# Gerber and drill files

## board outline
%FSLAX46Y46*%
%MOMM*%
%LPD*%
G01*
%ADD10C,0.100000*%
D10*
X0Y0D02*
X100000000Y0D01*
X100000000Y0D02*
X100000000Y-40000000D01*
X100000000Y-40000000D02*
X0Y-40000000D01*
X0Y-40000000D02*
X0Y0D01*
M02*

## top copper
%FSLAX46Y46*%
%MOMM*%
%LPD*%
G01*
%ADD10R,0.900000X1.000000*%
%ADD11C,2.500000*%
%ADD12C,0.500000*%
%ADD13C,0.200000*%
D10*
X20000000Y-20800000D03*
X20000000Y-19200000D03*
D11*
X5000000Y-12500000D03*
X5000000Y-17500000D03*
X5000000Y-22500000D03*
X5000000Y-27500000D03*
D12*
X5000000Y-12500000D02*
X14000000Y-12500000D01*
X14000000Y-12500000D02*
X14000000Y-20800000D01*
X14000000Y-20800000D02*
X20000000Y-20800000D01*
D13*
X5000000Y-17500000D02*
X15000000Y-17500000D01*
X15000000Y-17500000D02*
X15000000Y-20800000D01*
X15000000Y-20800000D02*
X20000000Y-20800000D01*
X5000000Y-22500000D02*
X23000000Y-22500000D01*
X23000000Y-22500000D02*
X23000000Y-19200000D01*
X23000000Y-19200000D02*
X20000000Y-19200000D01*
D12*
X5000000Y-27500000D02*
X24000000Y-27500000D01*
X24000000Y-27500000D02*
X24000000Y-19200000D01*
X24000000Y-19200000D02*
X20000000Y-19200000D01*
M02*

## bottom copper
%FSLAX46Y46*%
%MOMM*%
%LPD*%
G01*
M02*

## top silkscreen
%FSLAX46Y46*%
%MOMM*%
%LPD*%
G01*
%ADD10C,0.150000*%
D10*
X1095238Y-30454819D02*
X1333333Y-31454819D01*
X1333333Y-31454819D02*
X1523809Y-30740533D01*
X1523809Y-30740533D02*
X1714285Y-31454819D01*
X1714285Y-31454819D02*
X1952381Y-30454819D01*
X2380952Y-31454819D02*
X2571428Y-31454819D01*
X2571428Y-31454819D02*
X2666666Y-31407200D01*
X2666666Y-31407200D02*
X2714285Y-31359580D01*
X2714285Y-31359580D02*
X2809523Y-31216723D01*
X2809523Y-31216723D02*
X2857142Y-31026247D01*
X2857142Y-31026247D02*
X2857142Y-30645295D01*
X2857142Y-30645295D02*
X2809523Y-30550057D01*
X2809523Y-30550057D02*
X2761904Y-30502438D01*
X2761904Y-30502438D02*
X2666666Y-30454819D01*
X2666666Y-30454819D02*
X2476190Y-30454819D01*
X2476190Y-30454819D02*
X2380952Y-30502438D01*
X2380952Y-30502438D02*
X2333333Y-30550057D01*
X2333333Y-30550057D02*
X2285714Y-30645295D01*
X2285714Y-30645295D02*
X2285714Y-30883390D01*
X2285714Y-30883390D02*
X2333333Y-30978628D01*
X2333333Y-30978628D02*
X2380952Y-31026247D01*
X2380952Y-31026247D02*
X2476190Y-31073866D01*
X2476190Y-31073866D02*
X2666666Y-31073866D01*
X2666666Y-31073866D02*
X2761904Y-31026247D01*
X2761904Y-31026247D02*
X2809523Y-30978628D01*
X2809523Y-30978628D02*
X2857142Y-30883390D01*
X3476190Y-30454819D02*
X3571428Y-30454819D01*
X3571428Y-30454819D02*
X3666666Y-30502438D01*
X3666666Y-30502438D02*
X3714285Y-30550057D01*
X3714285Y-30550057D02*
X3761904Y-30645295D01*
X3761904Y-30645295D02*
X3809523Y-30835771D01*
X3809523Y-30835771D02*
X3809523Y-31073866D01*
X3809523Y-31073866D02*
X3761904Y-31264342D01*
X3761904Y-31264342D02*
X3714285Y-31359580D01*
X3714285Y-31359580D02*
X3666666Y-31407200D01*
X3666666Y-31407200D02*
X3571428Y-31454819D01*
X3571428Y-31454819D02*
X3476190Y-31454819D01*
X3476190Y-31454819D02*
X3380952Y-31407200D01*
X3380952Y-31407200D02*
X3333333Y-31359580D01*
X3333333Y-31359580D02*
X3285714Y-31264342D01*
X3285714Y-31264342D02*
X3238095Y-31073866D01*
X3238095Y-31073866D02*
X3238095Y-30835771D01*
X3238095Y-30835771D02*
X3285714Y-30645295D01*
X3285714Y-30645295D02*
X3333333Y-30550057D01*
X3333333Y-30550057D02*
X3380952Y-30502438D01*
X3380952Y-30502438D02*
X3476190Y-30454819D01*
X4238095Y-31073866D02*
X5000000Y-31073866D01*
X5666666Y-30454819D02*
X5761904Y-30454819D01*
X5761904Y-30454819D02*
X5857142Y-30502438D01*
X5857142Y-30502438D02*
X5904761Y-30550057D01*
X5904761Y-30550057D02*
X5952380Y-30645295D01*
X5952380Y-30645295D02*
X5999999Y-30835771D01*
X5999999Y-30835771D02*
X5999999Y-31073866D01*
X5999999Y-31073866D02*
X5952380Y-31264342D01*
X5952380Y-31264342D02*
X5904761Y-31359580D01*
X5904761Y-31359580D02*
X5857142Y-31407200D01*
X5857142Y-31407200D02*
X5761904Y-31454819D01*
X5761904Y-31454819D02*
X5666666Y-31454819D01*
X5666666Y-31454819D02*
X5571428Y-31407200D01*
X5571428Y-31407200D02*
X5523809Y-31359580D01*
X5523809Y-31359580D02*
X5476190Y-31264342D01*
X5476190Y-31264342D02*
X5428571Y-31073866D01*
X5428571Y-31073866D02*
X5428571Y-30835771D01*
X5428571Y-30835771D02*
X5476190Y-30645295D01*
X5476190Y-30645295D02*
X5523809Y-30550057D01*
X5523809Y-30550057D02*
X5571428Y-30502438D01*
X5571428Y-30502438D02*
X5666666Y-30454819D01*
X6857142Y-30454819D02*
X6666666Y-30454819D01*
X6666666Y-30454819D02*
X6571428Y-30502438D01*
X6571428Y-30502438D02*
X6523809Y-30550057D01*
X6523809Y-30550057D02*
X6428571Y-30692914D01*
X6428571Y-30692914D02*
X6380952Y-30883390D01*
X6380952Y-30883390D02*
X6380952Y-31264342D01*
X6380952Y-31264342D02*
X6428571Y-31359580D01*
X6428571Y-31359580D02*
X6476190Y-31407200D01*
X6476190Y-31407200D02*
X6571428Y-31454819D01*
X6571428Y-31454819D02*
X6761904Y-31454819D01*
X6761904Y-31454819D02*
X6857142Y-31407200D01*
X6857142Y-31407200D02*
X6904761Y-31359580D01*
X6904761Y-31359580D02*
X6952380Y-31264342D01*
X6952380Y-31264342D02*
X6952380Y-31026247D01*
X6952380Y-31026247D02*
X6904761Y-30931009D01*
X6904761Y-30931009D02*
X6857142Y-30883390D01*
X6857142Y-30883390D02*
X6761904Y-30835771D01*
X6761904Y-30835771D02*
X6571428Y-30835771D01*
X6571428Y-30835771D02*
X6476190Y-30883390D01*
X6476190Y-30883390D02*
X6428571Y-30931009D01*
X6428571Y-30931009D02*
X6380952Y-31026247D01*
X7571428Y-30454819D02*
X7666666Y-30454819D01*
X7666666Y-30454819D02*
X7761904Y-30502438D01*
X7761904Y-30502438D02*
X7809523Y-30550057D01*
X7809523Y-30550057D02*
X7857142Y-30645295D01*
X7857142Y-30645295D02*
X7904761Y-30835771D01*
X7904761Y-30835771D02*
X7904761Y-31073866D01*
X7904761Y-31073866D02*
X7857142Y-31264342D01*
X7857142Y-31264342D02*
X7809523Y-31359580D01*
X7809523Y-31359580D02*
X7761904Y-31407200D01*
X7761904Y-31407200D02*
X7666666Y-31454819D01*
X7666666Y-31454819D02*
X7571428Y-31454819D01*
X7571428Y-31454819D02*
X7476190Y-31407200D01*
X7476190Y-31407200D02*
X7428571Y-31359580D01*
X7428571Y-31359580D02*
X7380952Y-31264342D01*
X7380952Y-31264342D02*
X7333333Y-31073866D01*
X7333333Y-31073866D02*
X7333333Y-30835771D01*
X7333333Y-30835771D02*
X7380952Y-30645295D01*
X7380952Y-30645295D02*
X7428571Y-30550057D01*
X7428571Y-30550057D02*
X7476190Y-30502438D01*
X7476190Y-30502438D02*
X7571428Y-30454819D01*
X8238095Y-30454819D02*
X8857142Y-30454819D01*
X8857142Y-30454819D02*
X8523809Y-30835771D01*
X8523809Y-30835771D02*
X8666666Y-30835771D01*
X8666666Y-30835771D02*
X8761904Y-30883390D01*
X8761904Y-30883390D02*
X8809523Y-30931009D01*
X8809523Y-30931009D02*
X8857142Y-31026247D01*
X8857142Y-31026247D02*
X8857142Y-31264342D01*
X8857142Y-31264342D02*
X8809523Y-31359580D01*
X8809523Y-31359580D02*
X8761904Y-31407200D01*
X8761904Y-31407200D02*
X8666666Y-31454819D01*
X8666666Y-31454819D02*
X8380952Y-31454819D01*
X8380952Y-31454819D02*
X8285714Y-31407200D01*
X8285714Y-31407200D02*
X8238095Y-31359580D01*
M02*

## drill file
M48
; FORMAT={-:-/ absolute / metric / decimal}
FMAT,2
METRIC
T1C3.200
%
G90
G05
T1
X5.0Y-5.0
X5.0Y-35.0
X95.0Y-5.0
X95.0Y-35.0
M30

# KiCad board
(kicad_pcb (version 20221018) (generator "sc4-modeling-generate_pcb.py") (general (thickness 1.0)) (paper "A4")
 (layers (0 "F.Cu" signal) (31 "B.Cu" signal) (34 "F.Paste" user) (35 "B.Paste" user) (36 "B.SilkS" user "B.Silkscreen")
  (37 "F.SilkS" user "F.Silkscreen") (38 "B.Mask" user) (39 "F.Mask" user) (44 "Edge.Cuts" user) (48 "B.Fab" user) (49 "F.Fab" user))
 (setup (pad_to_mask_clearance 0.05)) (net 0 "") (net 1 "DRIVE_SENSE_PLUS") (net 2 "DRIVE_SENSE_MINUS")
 (gr_line (start 0.0 0.0) (end 100.0 0.0) (layer "Edge.Cuts") (width 0.1))
 (gr_line (start 100.0 0.0) (end 100.0 40.0) (layer "Edge.Cuts") (width 0.1))
 (gr_line (start 100.0 40.0) (end 0.0 40.0) (layer "Edge.Cuts") (width 0.1))
 (gr_line (start 0.0 40.0) (end 0.0 0.0) (layer "Edge.Cuts") (width 0.1))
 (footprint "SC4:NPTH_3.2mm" (layer "F.Cu") (at 5.0 5.0)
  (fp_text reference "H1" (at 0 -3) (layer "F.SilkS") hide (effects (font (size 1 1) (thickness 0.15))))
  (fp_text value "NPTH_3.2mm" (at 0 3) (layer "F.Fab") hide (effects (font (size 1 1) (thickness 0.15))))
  (pad "1" np_thru_hole circle (at 0 0) (size 3.2 3.2) (drill 3.2) (layers "*.Cu" "*.Mask")))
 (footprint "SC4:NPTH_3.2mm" (layer "F.Cu") (at 95.0 5.0)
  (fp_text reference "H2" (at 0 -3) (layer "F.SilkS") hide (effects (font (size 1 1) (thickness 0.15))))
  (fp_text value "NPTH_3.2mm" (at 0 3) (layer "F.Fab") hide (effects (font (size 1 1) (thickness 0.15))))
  (pad "1" np_thru_hole circle (at 0 0) (size 3.2 3.2) (drill 3.2) (layers "*.Cu" "*.Mask")))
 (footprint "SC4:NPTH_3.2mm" (layer "F.Cu") (at 5.0 35.0)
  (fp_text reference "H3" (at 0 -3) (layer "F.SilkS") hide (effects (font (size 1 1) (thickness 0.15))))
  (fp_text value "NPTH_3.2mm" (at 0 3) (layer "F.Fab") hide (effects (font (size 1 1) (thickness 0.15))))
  (pad "1" np_thru_hole circle (at 0 0) (size 3.2 3.2) (drill 3.2) (layers "*.Cu" "*.Mask")))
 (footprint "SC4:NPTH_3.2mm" (layer "F.Cu") (at 95.0 35.0)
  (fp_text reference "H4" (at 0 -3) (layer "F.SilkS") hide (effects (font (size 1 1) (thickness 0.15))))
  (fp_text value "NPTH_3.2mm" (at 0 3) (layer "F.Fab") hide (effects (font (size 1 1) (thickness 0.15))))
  (pad "1" np_thru_hole circle (at 0 0) (size 3.2 3.2) (drill 3.2) (layers "*.Cu" "*.Mask")))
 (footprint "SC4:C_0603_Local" (layer "F.Cu") (at 20.0 20.0 90)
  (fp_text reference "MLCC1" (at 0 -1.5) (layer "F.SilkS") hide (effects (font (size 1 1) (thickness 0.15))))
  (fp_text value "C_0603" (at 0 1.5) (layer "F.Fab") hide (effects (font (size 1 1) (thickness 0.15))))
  (pad "1" smd rect (at -0.8 0) (size 0.9 1.0) (layers "F.Cu" "F.Paste" "F.Mask") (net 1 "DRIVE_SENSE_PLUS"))
  (pad "2" smd rect (at 0.8 0) (size 0.9 1.0) (layers "F.Cu" "F.Paste" "F.Mask") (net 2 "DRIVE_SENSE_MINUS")))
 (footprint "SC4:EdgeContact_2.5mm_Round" (layer "F.Cu") (at 5.0 12.5)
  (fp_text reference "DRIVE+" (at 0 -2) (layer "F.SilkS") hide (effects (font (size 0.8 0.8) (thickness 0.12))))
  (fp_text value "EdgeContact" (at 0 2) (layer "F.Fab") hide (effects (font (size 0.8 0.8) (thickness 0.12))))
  (pad "1" smd circle (at 0 0) (size 2.5 2.5) (layers "F.Cu" "F.Mask") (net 1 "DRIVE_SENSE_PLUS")))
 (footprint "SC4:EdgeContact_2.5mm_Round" (layer "F.Cu") (at 5.0 17.5)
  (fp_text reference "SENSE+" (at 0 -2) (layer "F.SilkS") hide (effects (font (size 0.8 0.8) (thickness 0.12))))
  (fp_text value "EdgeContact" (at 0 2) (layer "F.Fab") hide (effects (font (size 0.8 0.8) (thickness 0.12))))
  (pad "1" smd circle (at 0 0) (size 2.5 2.5) (layers "F.Cu" "F.Mask") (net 1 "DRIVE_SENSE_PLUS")))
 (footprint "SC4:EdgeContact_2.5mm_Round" (layer "F.Cu") (at 5.0 22.5)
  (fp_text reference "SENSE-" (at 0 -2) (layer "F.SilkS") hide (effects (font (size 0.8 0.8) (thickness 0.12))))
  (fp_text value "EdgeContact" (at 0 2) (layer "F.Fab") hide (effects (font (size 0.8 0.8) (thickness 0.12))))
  (pad "1" smd circle (at 0 0) (size 2.5 2.5) (layers "F.Cu" "F.Mask") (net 2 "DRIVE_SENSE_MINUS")))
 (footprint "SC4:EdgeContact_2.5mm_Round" (layer "F.Cu") (at 5.0 27.5)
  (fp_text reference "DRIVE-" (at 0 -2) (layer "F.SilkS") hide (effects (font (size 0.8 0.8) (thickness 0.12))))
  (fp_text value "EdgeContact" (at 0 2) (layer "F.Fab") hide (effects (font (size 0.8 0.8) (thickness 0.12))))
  (pad "1" smd circle (at 0 0) (size 2.5 2.5) (layers "F.Cu" "F.Mask") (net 2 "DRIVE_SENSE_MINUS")))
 (segment (start 5.0 12.5) (end 14.0 12.5) (width 0.5) (layer "F.Cu") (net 1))
 (segment (start 14.0 12.5) (end 14.0 20.8) (width 0.5) (layer "F.Cu") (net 1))
 (segment (start 14.0 20.8) (end 20.0 20.8) (width 0.5) (layer "F.Cu") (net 1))
 (segment (start 5.0 17.5) (end 15.0 17.5) (width 0.2) (layer "F.Cu") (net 1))
 (segment (start 15.0 17.5) (end 15.0 20.8) (width 0.2) (layer "F.Cu") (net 1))
 (segment (start 15.0 20.8) (end 20.0 20.8) (width 0.2) (layer "F.Cu") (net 1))
 (segment (start 5.0 22.5) (end 23.0 22.5) (width 0.2) (layer "F.Cu") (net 2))
 (segment (start 23.0 22.5) (end 23.0 19.2) (width 0.2) (layer "F.Cu") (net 2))
 (segment (start 23.0 19.2) (end 20.0 19.2) (width 0.2) (layer "F.Cu") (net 2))
 (segment (start 5.0 27.5) (end 24.0 27.5) (width 0.5) (layer "F.Cu") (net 2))
 (segment (start 24.0 27.5) (end 24.0 19.2) (width 0.5) (layer "F.Cu") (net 2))
 (segment (start 24.0 19.2) (end 20.0 19.2) (width 0.5) (layer "F.Cu") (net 2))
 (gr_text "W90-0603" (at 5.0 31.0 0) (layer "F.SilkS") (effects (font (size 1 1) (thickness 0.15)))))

